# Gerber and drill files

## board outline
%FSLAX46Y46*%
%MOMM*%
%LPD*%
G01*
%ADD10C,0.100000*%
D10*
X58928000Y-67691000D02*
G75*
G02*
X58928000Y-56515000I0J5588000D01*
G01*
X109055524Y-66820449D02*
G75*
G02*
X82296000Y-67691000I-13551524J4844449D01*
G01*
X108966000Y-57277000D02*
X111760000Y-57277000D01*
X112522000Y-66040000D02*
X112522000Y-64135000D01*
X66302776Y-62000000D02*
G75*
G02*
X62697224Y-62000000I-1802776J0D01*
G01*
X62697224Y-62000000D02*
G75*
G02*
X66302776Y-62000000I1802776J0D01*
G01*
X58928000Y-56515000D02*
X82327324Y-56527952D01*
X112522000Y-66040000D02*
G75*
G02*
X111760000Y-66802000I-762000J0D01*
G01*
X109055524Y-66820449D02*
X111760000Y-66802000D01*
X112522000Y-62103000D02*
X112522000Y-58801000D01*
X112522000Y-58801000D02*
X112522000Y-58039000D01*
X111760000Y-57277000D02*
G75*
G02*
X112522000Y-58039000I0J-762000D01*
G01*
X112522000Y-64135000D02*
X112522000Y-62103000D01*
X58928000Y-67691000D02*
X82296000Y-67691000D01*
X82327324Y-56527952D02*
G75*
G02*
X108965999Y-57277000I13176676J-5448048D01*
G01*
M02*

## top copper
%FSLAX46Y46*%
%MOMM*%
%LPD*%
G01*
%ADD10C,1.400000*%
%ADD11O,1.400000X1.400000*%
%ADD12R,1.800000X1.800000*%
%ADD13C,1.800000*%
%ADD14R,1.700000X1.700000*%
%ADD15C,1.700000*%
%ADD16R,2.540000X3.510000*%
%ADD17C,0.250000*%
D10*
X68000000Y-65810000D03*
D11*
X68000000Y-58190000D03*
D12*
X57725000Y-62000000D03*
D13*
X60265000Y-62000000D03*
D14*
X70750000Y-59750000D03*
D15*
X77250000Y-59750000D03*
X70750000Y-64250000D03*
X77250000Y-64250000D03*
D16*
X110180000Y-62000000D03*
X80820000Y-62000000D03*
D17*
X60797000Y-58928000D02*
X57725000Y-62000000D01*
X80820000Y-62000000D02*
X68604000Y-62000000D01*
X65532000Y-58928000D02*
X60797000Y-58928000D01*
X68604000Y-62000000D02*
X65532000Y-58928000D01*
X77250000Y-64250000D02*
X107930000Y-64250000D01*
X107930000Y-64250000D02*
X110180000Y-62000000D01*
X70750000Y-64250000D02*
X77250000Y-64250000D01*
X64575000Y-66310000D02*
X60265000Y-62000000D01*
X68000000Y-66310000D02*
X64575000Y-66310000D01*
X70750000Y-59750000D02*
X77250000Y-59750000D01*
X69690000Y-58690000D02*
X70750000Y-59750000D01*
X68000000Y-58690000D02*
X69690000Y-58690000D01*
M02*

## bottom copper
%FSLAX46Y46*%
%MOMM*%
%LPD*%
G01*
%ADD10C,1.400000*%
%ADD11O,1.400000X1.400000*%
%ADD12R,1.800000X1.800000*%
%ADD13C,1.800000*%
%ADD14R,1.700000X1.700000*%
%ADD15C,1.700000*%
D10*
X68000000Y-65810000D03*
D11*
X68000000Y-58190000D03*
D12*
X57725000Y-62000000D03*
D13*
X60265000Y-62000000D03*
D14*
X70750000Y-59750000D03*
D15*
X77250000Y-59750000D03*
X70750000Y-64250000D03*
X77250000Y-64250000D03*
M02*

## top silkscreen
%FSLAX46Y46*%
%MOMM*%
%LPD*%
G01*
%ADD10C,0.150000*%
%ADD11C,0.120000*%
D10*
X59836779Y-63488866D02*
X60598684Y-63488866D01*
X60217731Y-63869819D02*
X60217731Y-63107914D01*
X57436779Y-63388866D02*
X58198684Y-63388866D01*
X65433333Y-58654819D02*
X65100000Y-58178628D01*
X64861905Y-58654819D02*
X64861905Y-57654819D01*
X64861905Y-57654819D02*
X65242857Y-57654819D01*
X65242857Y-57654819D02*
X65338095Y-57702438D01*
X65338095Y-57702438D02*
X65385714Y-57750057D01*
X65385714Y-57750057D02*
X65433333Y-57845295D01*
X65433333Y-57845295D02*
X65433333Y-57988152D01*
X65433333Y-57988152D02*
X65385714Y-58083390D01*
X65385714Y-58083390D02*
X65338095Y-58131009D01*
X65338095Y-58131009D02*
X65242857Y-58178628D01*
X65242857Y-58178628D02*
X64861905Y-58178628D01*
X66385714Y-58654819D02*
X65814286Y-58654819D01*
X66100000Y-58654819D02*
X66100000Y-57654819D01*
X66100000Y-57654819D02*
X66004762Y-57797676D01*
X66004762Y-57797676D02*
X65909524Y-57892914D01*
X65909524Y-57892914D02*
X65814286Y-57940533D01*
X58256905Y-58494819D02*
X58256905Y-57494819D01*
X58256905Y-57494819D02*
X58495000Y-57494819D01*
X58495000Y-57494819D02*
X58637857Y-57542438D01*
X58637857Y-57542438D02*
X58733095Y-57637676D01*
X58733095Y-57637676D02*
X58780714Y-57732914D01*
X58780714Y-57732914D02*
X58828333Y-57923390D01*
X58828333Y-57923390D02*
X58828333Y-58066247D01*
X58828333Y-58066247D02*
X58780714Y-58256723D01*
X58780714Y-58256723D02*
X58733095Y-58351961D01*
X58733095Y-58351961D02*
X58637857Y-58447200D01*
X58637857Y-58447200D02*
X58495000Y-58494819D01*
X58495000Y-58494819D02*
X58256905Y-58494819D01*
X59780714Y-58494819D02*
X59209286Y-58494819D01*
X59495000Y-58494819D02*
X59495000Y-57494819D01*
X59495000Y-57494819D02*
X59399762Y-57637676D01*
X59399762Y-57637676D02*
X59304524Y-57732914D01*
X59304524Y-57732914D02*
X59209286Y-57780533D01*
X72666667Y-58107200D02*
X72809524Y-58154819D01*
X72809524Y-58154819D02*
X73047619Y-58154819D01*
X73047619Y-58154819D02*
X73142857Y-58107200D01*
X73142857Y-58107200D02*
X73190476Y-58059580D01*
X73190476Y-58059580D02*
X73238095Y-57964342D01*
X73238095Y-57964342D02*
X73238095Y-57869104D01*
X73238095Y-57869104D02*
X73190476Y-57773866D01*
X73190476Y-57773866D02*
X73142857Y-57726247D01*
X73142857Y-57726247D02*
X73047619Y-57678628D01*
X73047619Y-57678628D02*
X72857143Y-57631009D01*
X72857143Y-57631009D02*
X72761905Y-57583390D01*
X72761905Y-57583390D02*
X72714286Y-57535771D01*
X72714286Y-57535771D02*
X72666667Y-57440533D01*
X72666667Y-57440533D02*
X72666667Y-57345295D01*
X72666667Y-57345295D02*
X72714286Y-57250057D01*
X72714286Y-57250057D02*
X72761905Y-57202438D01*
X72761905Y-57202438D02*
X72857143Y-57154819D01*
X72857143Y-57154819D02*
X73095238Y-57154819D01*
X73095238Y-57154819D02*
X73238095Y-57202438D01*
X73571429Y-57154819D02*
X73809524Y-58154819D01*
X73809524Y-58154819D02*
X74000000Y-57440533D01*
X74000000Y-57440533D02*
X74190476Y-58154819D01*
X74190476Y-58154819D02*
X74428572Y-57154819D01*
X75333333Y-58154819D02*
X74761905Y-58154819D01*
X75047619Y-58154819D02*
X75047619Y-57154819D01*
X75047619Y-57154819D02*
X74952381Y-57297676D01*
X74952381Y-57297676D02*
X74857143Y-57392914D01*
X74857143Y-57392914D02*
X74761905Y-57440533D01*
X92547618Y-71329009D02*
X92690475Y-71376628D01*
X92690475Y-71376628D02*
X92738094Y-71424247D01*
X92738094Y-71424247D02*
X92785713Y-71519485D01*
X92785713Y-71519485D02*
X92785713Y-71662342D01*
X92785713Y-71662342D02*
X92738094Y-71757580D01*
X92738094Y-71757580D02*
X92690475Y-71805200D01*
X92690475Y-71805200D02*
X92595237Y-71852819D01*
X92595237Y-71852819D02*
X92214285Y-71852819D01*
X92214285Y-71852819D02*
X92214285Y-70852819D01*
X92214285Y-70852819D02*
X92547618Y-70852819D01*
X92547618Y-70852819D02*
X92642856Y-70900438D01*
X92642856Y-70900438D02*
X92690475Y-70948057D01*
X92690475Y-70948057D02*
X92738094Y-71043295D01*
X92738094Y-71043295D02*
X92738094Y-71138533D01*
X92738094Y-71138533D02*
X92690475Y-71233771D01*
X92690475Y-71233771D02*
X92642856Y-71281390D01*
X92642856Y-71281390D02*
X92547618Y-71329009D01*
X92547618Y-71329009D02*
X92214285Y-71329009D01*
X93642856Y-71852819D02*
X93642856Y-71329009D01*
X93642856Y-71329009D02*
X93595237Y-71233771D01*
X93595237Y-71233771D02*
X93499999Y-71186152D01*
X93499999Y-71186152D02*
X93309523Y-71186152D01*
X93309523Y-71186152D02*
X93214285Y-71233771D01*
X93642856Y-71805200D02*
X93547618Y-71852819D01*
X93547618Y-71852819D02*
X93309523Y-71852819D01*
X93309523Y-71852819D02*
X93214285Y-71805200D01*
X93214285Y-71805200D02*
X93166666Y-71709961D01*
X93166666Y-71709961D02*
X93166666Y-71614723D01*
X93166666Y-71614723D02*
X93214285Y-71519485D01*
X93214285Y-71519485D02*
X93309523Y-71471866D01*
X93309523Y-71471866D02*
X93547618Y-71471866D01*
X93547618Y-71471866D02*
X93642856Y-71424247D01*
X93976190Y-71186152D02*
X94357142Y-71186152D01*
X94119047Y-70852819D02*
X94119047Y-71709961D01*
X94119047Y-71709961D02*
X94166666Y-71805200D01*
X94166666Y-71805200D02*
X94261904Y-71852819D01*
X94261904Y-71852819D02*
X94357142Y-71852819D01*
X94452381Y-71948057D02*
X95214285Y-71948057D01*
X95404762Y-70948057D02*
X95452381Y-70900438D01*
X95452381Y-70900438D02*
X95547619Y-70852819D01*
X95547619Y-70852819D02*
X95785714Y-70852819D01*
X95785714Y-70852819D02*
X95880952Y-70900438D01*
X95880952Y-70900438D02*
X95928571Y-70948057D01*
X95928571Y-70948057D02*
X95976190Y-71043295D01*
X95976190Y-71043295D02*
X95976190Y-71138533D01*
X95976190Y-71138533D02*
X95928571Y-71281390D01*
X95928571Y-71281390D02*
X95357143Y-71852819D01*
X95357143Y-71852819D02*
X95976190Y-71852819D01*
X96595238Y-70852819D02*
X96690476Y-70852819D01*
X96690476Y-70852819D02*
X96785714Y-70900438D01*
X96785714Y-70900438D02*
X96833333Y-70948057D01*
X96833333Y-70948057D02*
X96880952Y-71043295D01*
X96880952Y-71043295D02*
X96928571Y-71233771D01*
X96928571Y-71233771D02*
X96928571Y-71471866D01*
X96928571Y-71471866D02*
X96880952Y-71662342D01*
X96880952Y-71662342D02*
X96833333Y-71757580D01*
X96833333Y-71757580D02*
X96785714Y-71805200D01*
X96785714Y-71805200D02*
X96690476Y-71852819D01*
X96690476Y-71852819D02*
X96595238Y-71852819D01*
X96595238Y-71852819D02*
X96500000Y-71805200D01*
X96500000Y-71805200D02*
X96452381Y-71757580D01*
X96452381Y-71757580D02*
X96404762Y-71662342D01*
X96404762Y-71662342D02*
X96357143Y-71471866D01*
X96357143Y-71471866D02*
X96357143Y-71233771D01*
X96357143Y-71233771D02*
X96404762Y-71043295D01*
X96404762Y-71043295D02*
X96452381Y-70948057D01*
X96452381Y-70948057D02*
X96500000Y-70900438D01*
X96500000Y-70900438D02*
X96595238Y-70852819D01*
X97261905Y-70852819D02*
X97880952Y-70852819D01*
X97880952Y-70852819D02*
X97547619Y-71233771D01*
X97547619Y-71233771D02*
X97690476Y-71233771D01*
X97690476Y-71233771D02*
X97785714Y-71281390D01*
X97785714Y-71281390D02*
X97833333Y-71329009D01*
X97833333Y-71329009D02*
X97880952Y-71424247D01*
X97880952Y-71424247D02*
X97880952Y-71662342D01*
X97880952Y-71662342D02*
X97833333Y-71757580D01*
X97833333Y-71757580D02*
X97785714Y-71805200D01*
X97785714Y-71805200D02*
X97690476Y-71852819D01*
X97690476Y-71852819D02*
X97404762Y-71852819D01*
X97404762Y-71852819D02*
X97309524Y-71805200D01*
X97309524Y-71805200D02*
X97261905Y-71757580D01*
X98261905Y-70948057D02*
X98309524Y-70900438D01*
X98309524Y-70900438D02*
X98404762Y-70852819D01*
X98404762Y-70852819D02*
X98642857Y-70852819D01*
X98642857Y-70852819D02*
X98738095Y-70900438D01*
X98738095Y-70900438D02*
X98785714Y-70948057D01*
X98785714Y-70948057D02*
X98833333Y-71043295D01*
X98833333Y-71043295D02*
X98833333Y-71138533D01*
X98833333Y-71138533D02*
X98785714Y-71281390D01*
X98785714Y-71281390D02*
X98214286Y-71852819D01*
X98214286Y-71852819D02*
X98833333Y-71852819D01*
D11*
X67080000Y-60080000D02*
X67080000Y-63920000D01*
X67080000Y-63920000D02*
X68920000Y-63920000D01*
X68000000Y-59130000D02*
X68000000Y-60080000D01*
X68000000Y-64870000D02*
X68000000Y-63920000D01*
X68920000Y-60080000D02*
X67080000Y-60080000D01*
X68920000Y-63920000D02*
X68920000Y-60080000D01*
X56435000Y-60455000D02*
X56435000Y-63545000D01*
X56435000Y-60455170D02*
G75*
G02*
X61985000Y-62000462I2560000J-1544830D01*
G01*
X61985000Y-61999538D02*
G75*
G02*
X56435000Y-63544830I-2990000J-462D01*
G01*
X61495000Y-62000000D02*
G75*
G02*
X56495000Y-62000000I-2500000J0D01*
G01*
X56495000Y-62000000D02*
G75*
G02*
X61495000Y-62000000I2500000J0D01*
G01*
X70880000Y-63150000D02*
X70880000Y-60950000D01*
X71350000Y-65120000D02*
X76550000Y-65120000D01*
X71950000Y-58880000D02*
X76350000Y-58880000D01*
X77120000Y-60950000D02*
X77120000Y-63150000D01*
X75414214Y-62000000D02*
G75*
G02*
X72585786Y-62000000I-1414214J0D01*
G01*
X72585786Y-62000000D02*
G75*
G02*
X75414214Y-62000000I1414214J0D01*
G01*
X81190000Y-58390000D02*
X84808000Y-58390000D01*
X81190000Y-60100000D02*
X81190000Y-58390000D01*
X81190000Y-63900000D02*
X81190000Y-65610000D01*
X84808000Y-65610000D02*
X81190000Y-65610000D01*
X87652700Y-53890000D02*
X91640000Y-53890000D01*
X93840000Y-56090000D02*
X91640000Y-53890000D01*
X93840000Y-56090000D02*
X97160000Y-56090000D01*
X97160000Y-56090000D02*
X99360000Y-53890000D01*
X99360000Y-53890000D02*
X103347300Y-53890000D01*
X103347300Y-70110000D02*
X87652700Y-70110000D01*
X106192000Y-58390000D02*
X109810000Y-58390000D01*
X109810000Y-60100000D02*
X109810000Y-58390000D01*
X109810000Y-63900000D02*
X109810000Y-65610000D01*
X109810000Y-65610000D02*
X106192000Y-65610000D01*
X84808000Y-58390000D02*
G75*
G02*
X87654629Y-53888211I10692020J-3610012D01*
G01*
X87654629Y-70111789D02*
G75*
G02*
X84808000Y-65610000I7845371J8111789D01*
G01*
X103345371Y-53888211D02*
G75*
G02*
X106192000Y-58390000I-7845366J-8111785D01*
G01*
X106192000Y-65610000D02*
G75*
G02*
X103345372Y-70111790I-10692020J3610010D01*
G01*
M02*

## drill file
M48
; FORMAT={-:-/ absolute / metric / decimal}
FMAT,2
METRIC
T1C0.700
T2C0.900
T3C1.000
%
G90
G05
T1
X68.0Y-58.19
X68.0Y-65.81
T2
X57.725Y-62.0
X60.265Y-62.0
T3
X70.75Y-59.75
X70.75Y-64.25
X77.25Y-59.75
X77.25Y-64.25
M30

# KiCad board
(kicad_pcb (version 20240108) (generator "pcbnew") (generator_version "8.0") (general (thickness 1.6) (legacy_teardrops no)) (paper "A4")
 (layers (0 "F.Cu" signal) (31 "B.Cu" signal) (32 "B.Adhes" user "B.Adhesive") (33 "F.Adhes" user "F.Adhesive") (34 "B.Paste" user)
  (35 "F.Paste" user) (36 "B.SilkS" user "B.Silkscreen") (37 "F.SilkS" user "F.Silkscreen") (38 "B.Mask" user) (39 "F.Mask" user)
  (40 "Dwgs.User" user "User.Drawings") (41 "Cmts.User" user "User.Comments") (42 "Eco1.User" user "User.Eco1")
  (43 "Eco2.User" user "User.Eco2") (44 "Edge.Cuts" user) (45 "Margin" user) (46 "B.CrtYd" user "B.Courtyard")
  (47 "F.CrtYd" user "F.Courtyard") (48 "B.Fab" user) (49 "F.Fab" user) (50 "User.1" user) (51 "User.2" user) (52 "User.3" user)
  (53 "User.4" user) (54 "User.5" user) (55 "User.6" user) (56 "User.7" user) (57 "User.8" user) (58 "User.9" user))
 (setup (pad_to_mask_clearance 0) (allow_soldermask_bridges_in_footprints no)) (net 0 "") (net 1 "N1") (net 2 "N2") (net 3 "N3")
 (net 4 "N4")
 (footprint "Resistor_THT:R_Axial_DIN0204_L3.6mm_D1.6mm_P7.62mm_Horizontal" (layer "F.Cu") (at 68 65.81 90)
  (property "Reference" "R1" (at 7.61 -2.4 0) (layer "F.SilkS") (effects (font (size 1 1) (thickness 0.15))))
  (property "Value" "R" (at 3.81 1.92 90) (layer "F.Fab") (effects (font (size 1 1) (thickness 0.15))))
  (fp_line (start 5.73 -0.92) (end 1.89 -0.92) (stroke (width 0.12) (type solid)) (layer "F.SilkS"))
  (fp_line (start 1.89 -0.92) (end 1.89 0.92) (stroke (width 0.12) (type solid)) (layer "F.SilkS"))
  (fp_line (start 6.68 0) (end 5.73 0) (stroke (width 0.12) (type solid)) (layer "F.SilkS"))
  (fp_line (start 0.94 0) (end 1.89 0) (stroke (width 0.12) (type solid)) (layer "F.SilkS"))
  (fp_line (start 5.73 0.92) (end 5.73 -0.92) (stroke (width 0.12) (type solid)) (layer "F.SilkS"))
  (fp_line (start 1.89 0.92) (end 5.73 0.92) (stroke (width 0.12) (type solid)) (layer "F.SilkS"))
  (pad "1" thru_hole circle (at 0 0 90) (size 1.4 1.4) (drill 0.7) (layers "*.Cu" "*.Mask") (remove_unused_layers no) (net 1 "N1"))
  (pad "2" thru_hole oval (at 7.62 0 90) (size 1.4 1.4) (drill 0.7) (layers "*.Cu" "*.Mask") (remove_unused_layers no) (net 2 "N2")))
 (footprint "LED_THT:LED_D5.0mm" (layer "F.Cu") (at 57.725 62)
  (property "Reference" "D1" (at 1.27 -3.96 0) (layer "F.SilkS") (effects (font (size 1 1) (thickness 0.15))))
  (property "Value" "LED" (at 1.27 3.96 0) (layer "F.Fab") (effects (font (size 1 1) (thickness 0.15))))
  (fp_line (start -1.29 -1.545) (end -1.29 1.545) (stroke (width 0.12) (type solid)) (layer "F.SilkS"))
  (fp_arc (start -1.29 -1.54483) (mid 2.072002 -2.880433) (end 4.26 0.000462) (stroke (width 0.12) (type solid)) (layer "F.SilkS"))
  (fp_arc (start 4.26 -0.000462) (mid 2.072002 2.880433) (end -1.29 1.54483) (stroke (width 0.12) (type solid)) (layer "F.SilkS"))
  (fp_circle (center 1.27 0) (end 3.77 0) (stroke (width 0.12) (type solid)) (fill none) (layer "F.SilkS"))
  (pad "1" thru_hole rect (at 0 0) (size 1.8 1.8) (drill 0.9) (layers "*.Cu" "*.Mask") (remove_unused_layers no) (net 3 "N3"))
  (pad "2" thru_hole circle (at 2.54 0) (size 1.8 1.8) (drill 0.9) (layers "*.Cu" "*.Mask") (remove_unused_layers no) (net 1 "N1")))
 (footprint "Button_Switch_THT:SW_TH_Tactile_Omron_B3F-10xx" (layer "F.Cu") (at 70.75 59.75)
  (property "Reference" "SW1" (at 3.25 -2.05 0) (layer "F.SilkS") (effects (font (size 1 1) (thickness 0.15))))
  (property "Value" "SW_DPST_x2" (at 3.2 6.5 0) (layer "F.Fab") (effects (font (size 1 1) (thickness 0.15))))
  (fp_line (start 0.13 3.4) (end 0.13 1.2) (stroke (width 0.12) (type solid)) (layer "F.SilkS"))
  (fp_line (start 0.6 5.37) (end 5.8 5.37) (stroke (width 0.12) (type solid)) (layer "F.SilkS"))
  (fp_line (start 1.2 -0.87) (end 5.6 -0.87) (stroke (width 0.12) (type solid)) (layer "F.SilkS"))
  (fp_line (start 6.37 1.2) (end 6.37 3.4) (stroke (width 0.12) (type solid)) (layer "F.SilkS"))
  (fp_circle (center 3.25 2.25) (end 4.25 3.25) (stroke (width 0.12) (type solid)) (fill none) (layer "F.SilkS"))
  (pad "1" thru_hole rect (at 0 0) (size 1.7 1.7) (drill 1) (layers "*.Cu" "*.Mask") (remove_unused_layers no) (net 2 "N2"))
  (pad "1" thru_hole circle (at 6.5 0) (size 1.7 1.7) (drill 1) (layers "*.Cu" "*.Mask") (remove_unused_layers no) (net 2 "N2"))
  (pad "2" thru_hole circle (at 0 4.5) (size 1.7 1.7) (drill 1) (layers "*.Cu" "*.Mask") (remove_unused_layers no) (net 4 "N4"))
  (pad "2" thru_hole circle (at 6.5 4.5) (size 1.7 1.7) (drill 1) (layers "*.Cu" "*.Mask") (remove_unused_layers no) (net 4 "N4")))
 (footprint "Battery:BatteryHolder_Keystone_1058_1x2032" (layer "F.Cu") (at 95.5 62 180)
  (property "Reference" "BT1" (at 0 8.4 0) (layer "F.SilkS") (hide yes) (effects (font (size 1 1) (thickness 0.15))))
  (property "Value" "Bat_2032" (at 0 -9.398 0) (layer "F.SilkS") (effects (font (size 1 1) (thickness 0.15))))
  (fp_line (start 14.31 3.61) (end 10.692 3.61) (stroke (width 0.12) (type solid)) (layer "F.SilkS"))
  (fp_line (start 14.31 1.9) (end 14.31 3.61) (stroke (width 0.12) (type solid)) (layer "F.SilkS"))
  (fp_line (start 14.31 -1.9) (end 14.31 -3.61) (stroke (width 0.12) (type solid)) (layer "F.SilkS"))
  (fp_line (start 10.692 -3.61) (end 14.31 -3.61) (stroke (width 0.12) (type solid)) (layer "F.SilkS"))
  (fp_line (start 7.8473 8.11) (end 3.86 8.11) (stroke (width 0.12) (type solid)) (layer "F.SilkS"))
  (fp_line (start 1.66 5.91) (end 3.86 8.11) (stroke (width 0.12) (type solid)) (layer "F.SilkS"))
  (fp_line (start 1.66 5.91) (end -1.66 5.91) (stroke (width 0.12) (type solid)) (layer "F.SilkS"))
  (fp_line (start -1.66 5.91) (end -3.86 8.11) (stroke (width 0.12) (type solid)) (layer "F.SilkS"))
  (fp_line (start -3.86 8.11) (end -7.8473 8.11) (stroke (width 0.12) (type solid)) (layer "F.SilkS"))
  (fp_line (start -7.8473 -8.11) (end 7.8473 -8.11) (stroke (width 0.12) (type solid)) (layer "F.SilkS"))
  (fp_line (start -10.692 3.61) (end -14.31 3.61) (stroke (width 0.12) (type solid)) (layer "F.SilkS"))
  (fp_line (start -14.31 1.9) (end -14.31 3.61) (stroke (width 0.12) (type solid)) (layer "F.SilkS"))
  (fp_line (start -14.31 -1.9) (end -14.31 -3.61) (stroke (width 0.12) (type solid)) (layer "F.SilkS"))
  (fp_line (start -14.31 -3.61) (end -10.692 -3.61) (stroke (width 0.12) (type solid)) (layer "F.SilkS"))
  (fp_arc (start 10.692 3.61) (mid 9.538084 6.031244) (end 7.845371 8.111789) (stroke (width 0.12) (type solid)) (layer "F.SilkS"))
  (fp_arc (start 7.845371 -8.111789) (mid 9.538085 -6.031244) (end 10.692 -3.61) (stroke (width 0.12) (type solid)) (layer "F.SilkS"))
  (fp_arc (start -7.845371 8.111789) (mid -9.538085 6.031244) (end -10.692 3.61) (stroke (width 0.12) (type solid)) (layer "F.SilkS"))
  (fp_arc (start -10.692 -3.61) (mid -9.538084 -6.031244) (end -7.845371 -8.111789) (stroke (width 0.12) (type solid)) (layer "F.SilkS"))
  (pad "1" smd rect (at -14.68 0 180) (size 2.54 3.51) (layers "F.Cu" "F.Paste" "F.Mask") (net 4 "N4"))
  (pad "2" smd rect (at 14.68 0 180) (size 2.54 3.51) (layers "F.Cu" "F.Paste" "F.Mask") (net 3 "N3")))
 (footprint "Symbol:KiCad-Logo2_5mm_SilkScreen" (layer "B.Cu") (at 95.377 60.071 180)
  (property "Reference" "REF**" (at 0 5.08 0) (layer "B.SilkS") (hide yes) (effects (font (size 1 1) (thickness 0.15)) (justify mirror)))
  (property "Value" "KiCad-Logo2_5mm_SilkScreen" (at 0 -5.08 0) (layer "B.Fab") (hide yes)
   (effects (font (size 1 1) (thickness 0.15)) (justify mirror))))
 (gr_arc (start 58.928 67.691) (mid 53.34 62.103) (end 58.928 56.515) (locked yes) (stroke (width 0.1) (type default)) (layer "Edge.Cuts"))
 (gr_arc (start 109.055524 66.820449) (mid 95.971939 76.359794) (end 82.296 67.691) (locked yes) (stroke (width 0.1) (type default))
  (layer "Edge.Cuts"))
 (gr_line (start 108.966 57.277) (end 111.76 57.277) (locked yes) (stroke (width 0.1) (type default)) (layer "Edge.Cuts"))
 (gr_line (start 112.522 66.04) (end 112.522 64.135) (locked yes) (stroke (width 0.1) (type default)) (layer "Edge.Cuts"))
 (gr_circle (center 64.5 62) (end 65.5 63.5) (stroke (width 0.1) (type default)) (fill none) (layer "Edge.Cuts"))
 (gr_line (start 58.928 56.515) (end 82.327324 56.527952) (locked yes) (stroke (width 0.1) (type default)) (layer "Edge.Cuts"))
 (gr_arc (start 112.522 66.04) (mid 112.298815 66.578815) (end 111.76 66.802) (locked yes) (stroke (width 0.1) (type default))
  (layer "Edge.Cuts"))
 (gr_line (start 109.055524 66.820449) (end 111.76 66.802) (locked yes) (stroke (width 0.1) (type default)) (layer "Edge.Cuts"))
 (gr_line (start 112.522 62.103) (end 112.522 58.801) (locked yes) (stroke (width 0.1) (type default)) (layer "Edge.Cuts"))
 (gr_line (start 112.522 58.801) (end 112.522 58.039) (locked yes) (stroke (width 0.1) (type default)) (layer "Edge.Cuts"))
 (gr_arc (start 111.76 57.277) (mid 112.298815 57.500185) (end 112.522 58.039) (locked yes) (stroke (width 0.1) (type default))
  (layer "Edge.Cuts"))
 (gr_line (start 112.522 64.135) (end 112.522 62.103) (locked yes) (stroke (width 0.1) (type default)) (layer "Edge.Cuts"))
 (gr_line (start 58.928 67.691) (end 82.296 67.691) (locked yes) (stroke (width 0.1) (type default)) (layer "Edge.Cuts"))
 (gr_arc (start 82.327324 56.527952) (mid 95.904775 47.723092) (end 108.965999 57.277) (locked yes) (stroke (width 0.1) (type default))
  (layer "Edge.Cuts"))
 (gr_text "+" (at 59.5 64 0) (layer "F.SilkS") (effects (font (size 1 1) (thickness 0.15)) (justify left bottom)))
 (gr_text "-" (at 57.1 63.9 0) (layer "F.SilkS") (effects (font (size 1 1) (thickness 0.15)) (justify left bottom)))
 (segment (start 60.797 58.928) (end 57.725 62) (width 0.25) (layer "F.Cu") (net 3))
 (segment (start 80.82 62) (end 68.604 62) (width 0.25) (layer "F.Cu") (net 3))
 (segment (start 65.532 58.928) (end 60.797 58.928) (width 0.25) (layer "F.Cu") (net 3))
 (segment (start 68.604 62) (end 65.532 58.928) (width 0.25) (layer "F.Cu") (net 3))
 (segment (start 77.25 64.25) (end 107.93 64.25) (width 0.25) (layer "F.Cu") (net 4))
 (segment (start 107.93 64.25) (end 110.18 62) (width 0.25) (layer "F.Cu") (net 4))
 (segment (start 70.75 64.25) (end 77.25 64.25) (width 0.25) (layer "F.Cu") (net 4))
 (segment (start 64.575 66.31) (end 60.265 62) (width 0.25) (layer "F.Cu") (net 1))
 (segment (start 68 66.31) (end 64.575 66.31) (width 0.25) (layer "F.Cu") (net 1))
 (segment (start 70.75 59.75) (end 77.25 59.75) (width 0.25) (layer "F.Cu") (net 2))
 (segment (start 69.69 58.69) (end 70.75 59.75) (width 0.25) (layer "F.Cu") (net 2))
 (segment (start 68 58.69) (end 69.69 58.69) (width 0.25) (layer "F.Cu") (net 2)))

